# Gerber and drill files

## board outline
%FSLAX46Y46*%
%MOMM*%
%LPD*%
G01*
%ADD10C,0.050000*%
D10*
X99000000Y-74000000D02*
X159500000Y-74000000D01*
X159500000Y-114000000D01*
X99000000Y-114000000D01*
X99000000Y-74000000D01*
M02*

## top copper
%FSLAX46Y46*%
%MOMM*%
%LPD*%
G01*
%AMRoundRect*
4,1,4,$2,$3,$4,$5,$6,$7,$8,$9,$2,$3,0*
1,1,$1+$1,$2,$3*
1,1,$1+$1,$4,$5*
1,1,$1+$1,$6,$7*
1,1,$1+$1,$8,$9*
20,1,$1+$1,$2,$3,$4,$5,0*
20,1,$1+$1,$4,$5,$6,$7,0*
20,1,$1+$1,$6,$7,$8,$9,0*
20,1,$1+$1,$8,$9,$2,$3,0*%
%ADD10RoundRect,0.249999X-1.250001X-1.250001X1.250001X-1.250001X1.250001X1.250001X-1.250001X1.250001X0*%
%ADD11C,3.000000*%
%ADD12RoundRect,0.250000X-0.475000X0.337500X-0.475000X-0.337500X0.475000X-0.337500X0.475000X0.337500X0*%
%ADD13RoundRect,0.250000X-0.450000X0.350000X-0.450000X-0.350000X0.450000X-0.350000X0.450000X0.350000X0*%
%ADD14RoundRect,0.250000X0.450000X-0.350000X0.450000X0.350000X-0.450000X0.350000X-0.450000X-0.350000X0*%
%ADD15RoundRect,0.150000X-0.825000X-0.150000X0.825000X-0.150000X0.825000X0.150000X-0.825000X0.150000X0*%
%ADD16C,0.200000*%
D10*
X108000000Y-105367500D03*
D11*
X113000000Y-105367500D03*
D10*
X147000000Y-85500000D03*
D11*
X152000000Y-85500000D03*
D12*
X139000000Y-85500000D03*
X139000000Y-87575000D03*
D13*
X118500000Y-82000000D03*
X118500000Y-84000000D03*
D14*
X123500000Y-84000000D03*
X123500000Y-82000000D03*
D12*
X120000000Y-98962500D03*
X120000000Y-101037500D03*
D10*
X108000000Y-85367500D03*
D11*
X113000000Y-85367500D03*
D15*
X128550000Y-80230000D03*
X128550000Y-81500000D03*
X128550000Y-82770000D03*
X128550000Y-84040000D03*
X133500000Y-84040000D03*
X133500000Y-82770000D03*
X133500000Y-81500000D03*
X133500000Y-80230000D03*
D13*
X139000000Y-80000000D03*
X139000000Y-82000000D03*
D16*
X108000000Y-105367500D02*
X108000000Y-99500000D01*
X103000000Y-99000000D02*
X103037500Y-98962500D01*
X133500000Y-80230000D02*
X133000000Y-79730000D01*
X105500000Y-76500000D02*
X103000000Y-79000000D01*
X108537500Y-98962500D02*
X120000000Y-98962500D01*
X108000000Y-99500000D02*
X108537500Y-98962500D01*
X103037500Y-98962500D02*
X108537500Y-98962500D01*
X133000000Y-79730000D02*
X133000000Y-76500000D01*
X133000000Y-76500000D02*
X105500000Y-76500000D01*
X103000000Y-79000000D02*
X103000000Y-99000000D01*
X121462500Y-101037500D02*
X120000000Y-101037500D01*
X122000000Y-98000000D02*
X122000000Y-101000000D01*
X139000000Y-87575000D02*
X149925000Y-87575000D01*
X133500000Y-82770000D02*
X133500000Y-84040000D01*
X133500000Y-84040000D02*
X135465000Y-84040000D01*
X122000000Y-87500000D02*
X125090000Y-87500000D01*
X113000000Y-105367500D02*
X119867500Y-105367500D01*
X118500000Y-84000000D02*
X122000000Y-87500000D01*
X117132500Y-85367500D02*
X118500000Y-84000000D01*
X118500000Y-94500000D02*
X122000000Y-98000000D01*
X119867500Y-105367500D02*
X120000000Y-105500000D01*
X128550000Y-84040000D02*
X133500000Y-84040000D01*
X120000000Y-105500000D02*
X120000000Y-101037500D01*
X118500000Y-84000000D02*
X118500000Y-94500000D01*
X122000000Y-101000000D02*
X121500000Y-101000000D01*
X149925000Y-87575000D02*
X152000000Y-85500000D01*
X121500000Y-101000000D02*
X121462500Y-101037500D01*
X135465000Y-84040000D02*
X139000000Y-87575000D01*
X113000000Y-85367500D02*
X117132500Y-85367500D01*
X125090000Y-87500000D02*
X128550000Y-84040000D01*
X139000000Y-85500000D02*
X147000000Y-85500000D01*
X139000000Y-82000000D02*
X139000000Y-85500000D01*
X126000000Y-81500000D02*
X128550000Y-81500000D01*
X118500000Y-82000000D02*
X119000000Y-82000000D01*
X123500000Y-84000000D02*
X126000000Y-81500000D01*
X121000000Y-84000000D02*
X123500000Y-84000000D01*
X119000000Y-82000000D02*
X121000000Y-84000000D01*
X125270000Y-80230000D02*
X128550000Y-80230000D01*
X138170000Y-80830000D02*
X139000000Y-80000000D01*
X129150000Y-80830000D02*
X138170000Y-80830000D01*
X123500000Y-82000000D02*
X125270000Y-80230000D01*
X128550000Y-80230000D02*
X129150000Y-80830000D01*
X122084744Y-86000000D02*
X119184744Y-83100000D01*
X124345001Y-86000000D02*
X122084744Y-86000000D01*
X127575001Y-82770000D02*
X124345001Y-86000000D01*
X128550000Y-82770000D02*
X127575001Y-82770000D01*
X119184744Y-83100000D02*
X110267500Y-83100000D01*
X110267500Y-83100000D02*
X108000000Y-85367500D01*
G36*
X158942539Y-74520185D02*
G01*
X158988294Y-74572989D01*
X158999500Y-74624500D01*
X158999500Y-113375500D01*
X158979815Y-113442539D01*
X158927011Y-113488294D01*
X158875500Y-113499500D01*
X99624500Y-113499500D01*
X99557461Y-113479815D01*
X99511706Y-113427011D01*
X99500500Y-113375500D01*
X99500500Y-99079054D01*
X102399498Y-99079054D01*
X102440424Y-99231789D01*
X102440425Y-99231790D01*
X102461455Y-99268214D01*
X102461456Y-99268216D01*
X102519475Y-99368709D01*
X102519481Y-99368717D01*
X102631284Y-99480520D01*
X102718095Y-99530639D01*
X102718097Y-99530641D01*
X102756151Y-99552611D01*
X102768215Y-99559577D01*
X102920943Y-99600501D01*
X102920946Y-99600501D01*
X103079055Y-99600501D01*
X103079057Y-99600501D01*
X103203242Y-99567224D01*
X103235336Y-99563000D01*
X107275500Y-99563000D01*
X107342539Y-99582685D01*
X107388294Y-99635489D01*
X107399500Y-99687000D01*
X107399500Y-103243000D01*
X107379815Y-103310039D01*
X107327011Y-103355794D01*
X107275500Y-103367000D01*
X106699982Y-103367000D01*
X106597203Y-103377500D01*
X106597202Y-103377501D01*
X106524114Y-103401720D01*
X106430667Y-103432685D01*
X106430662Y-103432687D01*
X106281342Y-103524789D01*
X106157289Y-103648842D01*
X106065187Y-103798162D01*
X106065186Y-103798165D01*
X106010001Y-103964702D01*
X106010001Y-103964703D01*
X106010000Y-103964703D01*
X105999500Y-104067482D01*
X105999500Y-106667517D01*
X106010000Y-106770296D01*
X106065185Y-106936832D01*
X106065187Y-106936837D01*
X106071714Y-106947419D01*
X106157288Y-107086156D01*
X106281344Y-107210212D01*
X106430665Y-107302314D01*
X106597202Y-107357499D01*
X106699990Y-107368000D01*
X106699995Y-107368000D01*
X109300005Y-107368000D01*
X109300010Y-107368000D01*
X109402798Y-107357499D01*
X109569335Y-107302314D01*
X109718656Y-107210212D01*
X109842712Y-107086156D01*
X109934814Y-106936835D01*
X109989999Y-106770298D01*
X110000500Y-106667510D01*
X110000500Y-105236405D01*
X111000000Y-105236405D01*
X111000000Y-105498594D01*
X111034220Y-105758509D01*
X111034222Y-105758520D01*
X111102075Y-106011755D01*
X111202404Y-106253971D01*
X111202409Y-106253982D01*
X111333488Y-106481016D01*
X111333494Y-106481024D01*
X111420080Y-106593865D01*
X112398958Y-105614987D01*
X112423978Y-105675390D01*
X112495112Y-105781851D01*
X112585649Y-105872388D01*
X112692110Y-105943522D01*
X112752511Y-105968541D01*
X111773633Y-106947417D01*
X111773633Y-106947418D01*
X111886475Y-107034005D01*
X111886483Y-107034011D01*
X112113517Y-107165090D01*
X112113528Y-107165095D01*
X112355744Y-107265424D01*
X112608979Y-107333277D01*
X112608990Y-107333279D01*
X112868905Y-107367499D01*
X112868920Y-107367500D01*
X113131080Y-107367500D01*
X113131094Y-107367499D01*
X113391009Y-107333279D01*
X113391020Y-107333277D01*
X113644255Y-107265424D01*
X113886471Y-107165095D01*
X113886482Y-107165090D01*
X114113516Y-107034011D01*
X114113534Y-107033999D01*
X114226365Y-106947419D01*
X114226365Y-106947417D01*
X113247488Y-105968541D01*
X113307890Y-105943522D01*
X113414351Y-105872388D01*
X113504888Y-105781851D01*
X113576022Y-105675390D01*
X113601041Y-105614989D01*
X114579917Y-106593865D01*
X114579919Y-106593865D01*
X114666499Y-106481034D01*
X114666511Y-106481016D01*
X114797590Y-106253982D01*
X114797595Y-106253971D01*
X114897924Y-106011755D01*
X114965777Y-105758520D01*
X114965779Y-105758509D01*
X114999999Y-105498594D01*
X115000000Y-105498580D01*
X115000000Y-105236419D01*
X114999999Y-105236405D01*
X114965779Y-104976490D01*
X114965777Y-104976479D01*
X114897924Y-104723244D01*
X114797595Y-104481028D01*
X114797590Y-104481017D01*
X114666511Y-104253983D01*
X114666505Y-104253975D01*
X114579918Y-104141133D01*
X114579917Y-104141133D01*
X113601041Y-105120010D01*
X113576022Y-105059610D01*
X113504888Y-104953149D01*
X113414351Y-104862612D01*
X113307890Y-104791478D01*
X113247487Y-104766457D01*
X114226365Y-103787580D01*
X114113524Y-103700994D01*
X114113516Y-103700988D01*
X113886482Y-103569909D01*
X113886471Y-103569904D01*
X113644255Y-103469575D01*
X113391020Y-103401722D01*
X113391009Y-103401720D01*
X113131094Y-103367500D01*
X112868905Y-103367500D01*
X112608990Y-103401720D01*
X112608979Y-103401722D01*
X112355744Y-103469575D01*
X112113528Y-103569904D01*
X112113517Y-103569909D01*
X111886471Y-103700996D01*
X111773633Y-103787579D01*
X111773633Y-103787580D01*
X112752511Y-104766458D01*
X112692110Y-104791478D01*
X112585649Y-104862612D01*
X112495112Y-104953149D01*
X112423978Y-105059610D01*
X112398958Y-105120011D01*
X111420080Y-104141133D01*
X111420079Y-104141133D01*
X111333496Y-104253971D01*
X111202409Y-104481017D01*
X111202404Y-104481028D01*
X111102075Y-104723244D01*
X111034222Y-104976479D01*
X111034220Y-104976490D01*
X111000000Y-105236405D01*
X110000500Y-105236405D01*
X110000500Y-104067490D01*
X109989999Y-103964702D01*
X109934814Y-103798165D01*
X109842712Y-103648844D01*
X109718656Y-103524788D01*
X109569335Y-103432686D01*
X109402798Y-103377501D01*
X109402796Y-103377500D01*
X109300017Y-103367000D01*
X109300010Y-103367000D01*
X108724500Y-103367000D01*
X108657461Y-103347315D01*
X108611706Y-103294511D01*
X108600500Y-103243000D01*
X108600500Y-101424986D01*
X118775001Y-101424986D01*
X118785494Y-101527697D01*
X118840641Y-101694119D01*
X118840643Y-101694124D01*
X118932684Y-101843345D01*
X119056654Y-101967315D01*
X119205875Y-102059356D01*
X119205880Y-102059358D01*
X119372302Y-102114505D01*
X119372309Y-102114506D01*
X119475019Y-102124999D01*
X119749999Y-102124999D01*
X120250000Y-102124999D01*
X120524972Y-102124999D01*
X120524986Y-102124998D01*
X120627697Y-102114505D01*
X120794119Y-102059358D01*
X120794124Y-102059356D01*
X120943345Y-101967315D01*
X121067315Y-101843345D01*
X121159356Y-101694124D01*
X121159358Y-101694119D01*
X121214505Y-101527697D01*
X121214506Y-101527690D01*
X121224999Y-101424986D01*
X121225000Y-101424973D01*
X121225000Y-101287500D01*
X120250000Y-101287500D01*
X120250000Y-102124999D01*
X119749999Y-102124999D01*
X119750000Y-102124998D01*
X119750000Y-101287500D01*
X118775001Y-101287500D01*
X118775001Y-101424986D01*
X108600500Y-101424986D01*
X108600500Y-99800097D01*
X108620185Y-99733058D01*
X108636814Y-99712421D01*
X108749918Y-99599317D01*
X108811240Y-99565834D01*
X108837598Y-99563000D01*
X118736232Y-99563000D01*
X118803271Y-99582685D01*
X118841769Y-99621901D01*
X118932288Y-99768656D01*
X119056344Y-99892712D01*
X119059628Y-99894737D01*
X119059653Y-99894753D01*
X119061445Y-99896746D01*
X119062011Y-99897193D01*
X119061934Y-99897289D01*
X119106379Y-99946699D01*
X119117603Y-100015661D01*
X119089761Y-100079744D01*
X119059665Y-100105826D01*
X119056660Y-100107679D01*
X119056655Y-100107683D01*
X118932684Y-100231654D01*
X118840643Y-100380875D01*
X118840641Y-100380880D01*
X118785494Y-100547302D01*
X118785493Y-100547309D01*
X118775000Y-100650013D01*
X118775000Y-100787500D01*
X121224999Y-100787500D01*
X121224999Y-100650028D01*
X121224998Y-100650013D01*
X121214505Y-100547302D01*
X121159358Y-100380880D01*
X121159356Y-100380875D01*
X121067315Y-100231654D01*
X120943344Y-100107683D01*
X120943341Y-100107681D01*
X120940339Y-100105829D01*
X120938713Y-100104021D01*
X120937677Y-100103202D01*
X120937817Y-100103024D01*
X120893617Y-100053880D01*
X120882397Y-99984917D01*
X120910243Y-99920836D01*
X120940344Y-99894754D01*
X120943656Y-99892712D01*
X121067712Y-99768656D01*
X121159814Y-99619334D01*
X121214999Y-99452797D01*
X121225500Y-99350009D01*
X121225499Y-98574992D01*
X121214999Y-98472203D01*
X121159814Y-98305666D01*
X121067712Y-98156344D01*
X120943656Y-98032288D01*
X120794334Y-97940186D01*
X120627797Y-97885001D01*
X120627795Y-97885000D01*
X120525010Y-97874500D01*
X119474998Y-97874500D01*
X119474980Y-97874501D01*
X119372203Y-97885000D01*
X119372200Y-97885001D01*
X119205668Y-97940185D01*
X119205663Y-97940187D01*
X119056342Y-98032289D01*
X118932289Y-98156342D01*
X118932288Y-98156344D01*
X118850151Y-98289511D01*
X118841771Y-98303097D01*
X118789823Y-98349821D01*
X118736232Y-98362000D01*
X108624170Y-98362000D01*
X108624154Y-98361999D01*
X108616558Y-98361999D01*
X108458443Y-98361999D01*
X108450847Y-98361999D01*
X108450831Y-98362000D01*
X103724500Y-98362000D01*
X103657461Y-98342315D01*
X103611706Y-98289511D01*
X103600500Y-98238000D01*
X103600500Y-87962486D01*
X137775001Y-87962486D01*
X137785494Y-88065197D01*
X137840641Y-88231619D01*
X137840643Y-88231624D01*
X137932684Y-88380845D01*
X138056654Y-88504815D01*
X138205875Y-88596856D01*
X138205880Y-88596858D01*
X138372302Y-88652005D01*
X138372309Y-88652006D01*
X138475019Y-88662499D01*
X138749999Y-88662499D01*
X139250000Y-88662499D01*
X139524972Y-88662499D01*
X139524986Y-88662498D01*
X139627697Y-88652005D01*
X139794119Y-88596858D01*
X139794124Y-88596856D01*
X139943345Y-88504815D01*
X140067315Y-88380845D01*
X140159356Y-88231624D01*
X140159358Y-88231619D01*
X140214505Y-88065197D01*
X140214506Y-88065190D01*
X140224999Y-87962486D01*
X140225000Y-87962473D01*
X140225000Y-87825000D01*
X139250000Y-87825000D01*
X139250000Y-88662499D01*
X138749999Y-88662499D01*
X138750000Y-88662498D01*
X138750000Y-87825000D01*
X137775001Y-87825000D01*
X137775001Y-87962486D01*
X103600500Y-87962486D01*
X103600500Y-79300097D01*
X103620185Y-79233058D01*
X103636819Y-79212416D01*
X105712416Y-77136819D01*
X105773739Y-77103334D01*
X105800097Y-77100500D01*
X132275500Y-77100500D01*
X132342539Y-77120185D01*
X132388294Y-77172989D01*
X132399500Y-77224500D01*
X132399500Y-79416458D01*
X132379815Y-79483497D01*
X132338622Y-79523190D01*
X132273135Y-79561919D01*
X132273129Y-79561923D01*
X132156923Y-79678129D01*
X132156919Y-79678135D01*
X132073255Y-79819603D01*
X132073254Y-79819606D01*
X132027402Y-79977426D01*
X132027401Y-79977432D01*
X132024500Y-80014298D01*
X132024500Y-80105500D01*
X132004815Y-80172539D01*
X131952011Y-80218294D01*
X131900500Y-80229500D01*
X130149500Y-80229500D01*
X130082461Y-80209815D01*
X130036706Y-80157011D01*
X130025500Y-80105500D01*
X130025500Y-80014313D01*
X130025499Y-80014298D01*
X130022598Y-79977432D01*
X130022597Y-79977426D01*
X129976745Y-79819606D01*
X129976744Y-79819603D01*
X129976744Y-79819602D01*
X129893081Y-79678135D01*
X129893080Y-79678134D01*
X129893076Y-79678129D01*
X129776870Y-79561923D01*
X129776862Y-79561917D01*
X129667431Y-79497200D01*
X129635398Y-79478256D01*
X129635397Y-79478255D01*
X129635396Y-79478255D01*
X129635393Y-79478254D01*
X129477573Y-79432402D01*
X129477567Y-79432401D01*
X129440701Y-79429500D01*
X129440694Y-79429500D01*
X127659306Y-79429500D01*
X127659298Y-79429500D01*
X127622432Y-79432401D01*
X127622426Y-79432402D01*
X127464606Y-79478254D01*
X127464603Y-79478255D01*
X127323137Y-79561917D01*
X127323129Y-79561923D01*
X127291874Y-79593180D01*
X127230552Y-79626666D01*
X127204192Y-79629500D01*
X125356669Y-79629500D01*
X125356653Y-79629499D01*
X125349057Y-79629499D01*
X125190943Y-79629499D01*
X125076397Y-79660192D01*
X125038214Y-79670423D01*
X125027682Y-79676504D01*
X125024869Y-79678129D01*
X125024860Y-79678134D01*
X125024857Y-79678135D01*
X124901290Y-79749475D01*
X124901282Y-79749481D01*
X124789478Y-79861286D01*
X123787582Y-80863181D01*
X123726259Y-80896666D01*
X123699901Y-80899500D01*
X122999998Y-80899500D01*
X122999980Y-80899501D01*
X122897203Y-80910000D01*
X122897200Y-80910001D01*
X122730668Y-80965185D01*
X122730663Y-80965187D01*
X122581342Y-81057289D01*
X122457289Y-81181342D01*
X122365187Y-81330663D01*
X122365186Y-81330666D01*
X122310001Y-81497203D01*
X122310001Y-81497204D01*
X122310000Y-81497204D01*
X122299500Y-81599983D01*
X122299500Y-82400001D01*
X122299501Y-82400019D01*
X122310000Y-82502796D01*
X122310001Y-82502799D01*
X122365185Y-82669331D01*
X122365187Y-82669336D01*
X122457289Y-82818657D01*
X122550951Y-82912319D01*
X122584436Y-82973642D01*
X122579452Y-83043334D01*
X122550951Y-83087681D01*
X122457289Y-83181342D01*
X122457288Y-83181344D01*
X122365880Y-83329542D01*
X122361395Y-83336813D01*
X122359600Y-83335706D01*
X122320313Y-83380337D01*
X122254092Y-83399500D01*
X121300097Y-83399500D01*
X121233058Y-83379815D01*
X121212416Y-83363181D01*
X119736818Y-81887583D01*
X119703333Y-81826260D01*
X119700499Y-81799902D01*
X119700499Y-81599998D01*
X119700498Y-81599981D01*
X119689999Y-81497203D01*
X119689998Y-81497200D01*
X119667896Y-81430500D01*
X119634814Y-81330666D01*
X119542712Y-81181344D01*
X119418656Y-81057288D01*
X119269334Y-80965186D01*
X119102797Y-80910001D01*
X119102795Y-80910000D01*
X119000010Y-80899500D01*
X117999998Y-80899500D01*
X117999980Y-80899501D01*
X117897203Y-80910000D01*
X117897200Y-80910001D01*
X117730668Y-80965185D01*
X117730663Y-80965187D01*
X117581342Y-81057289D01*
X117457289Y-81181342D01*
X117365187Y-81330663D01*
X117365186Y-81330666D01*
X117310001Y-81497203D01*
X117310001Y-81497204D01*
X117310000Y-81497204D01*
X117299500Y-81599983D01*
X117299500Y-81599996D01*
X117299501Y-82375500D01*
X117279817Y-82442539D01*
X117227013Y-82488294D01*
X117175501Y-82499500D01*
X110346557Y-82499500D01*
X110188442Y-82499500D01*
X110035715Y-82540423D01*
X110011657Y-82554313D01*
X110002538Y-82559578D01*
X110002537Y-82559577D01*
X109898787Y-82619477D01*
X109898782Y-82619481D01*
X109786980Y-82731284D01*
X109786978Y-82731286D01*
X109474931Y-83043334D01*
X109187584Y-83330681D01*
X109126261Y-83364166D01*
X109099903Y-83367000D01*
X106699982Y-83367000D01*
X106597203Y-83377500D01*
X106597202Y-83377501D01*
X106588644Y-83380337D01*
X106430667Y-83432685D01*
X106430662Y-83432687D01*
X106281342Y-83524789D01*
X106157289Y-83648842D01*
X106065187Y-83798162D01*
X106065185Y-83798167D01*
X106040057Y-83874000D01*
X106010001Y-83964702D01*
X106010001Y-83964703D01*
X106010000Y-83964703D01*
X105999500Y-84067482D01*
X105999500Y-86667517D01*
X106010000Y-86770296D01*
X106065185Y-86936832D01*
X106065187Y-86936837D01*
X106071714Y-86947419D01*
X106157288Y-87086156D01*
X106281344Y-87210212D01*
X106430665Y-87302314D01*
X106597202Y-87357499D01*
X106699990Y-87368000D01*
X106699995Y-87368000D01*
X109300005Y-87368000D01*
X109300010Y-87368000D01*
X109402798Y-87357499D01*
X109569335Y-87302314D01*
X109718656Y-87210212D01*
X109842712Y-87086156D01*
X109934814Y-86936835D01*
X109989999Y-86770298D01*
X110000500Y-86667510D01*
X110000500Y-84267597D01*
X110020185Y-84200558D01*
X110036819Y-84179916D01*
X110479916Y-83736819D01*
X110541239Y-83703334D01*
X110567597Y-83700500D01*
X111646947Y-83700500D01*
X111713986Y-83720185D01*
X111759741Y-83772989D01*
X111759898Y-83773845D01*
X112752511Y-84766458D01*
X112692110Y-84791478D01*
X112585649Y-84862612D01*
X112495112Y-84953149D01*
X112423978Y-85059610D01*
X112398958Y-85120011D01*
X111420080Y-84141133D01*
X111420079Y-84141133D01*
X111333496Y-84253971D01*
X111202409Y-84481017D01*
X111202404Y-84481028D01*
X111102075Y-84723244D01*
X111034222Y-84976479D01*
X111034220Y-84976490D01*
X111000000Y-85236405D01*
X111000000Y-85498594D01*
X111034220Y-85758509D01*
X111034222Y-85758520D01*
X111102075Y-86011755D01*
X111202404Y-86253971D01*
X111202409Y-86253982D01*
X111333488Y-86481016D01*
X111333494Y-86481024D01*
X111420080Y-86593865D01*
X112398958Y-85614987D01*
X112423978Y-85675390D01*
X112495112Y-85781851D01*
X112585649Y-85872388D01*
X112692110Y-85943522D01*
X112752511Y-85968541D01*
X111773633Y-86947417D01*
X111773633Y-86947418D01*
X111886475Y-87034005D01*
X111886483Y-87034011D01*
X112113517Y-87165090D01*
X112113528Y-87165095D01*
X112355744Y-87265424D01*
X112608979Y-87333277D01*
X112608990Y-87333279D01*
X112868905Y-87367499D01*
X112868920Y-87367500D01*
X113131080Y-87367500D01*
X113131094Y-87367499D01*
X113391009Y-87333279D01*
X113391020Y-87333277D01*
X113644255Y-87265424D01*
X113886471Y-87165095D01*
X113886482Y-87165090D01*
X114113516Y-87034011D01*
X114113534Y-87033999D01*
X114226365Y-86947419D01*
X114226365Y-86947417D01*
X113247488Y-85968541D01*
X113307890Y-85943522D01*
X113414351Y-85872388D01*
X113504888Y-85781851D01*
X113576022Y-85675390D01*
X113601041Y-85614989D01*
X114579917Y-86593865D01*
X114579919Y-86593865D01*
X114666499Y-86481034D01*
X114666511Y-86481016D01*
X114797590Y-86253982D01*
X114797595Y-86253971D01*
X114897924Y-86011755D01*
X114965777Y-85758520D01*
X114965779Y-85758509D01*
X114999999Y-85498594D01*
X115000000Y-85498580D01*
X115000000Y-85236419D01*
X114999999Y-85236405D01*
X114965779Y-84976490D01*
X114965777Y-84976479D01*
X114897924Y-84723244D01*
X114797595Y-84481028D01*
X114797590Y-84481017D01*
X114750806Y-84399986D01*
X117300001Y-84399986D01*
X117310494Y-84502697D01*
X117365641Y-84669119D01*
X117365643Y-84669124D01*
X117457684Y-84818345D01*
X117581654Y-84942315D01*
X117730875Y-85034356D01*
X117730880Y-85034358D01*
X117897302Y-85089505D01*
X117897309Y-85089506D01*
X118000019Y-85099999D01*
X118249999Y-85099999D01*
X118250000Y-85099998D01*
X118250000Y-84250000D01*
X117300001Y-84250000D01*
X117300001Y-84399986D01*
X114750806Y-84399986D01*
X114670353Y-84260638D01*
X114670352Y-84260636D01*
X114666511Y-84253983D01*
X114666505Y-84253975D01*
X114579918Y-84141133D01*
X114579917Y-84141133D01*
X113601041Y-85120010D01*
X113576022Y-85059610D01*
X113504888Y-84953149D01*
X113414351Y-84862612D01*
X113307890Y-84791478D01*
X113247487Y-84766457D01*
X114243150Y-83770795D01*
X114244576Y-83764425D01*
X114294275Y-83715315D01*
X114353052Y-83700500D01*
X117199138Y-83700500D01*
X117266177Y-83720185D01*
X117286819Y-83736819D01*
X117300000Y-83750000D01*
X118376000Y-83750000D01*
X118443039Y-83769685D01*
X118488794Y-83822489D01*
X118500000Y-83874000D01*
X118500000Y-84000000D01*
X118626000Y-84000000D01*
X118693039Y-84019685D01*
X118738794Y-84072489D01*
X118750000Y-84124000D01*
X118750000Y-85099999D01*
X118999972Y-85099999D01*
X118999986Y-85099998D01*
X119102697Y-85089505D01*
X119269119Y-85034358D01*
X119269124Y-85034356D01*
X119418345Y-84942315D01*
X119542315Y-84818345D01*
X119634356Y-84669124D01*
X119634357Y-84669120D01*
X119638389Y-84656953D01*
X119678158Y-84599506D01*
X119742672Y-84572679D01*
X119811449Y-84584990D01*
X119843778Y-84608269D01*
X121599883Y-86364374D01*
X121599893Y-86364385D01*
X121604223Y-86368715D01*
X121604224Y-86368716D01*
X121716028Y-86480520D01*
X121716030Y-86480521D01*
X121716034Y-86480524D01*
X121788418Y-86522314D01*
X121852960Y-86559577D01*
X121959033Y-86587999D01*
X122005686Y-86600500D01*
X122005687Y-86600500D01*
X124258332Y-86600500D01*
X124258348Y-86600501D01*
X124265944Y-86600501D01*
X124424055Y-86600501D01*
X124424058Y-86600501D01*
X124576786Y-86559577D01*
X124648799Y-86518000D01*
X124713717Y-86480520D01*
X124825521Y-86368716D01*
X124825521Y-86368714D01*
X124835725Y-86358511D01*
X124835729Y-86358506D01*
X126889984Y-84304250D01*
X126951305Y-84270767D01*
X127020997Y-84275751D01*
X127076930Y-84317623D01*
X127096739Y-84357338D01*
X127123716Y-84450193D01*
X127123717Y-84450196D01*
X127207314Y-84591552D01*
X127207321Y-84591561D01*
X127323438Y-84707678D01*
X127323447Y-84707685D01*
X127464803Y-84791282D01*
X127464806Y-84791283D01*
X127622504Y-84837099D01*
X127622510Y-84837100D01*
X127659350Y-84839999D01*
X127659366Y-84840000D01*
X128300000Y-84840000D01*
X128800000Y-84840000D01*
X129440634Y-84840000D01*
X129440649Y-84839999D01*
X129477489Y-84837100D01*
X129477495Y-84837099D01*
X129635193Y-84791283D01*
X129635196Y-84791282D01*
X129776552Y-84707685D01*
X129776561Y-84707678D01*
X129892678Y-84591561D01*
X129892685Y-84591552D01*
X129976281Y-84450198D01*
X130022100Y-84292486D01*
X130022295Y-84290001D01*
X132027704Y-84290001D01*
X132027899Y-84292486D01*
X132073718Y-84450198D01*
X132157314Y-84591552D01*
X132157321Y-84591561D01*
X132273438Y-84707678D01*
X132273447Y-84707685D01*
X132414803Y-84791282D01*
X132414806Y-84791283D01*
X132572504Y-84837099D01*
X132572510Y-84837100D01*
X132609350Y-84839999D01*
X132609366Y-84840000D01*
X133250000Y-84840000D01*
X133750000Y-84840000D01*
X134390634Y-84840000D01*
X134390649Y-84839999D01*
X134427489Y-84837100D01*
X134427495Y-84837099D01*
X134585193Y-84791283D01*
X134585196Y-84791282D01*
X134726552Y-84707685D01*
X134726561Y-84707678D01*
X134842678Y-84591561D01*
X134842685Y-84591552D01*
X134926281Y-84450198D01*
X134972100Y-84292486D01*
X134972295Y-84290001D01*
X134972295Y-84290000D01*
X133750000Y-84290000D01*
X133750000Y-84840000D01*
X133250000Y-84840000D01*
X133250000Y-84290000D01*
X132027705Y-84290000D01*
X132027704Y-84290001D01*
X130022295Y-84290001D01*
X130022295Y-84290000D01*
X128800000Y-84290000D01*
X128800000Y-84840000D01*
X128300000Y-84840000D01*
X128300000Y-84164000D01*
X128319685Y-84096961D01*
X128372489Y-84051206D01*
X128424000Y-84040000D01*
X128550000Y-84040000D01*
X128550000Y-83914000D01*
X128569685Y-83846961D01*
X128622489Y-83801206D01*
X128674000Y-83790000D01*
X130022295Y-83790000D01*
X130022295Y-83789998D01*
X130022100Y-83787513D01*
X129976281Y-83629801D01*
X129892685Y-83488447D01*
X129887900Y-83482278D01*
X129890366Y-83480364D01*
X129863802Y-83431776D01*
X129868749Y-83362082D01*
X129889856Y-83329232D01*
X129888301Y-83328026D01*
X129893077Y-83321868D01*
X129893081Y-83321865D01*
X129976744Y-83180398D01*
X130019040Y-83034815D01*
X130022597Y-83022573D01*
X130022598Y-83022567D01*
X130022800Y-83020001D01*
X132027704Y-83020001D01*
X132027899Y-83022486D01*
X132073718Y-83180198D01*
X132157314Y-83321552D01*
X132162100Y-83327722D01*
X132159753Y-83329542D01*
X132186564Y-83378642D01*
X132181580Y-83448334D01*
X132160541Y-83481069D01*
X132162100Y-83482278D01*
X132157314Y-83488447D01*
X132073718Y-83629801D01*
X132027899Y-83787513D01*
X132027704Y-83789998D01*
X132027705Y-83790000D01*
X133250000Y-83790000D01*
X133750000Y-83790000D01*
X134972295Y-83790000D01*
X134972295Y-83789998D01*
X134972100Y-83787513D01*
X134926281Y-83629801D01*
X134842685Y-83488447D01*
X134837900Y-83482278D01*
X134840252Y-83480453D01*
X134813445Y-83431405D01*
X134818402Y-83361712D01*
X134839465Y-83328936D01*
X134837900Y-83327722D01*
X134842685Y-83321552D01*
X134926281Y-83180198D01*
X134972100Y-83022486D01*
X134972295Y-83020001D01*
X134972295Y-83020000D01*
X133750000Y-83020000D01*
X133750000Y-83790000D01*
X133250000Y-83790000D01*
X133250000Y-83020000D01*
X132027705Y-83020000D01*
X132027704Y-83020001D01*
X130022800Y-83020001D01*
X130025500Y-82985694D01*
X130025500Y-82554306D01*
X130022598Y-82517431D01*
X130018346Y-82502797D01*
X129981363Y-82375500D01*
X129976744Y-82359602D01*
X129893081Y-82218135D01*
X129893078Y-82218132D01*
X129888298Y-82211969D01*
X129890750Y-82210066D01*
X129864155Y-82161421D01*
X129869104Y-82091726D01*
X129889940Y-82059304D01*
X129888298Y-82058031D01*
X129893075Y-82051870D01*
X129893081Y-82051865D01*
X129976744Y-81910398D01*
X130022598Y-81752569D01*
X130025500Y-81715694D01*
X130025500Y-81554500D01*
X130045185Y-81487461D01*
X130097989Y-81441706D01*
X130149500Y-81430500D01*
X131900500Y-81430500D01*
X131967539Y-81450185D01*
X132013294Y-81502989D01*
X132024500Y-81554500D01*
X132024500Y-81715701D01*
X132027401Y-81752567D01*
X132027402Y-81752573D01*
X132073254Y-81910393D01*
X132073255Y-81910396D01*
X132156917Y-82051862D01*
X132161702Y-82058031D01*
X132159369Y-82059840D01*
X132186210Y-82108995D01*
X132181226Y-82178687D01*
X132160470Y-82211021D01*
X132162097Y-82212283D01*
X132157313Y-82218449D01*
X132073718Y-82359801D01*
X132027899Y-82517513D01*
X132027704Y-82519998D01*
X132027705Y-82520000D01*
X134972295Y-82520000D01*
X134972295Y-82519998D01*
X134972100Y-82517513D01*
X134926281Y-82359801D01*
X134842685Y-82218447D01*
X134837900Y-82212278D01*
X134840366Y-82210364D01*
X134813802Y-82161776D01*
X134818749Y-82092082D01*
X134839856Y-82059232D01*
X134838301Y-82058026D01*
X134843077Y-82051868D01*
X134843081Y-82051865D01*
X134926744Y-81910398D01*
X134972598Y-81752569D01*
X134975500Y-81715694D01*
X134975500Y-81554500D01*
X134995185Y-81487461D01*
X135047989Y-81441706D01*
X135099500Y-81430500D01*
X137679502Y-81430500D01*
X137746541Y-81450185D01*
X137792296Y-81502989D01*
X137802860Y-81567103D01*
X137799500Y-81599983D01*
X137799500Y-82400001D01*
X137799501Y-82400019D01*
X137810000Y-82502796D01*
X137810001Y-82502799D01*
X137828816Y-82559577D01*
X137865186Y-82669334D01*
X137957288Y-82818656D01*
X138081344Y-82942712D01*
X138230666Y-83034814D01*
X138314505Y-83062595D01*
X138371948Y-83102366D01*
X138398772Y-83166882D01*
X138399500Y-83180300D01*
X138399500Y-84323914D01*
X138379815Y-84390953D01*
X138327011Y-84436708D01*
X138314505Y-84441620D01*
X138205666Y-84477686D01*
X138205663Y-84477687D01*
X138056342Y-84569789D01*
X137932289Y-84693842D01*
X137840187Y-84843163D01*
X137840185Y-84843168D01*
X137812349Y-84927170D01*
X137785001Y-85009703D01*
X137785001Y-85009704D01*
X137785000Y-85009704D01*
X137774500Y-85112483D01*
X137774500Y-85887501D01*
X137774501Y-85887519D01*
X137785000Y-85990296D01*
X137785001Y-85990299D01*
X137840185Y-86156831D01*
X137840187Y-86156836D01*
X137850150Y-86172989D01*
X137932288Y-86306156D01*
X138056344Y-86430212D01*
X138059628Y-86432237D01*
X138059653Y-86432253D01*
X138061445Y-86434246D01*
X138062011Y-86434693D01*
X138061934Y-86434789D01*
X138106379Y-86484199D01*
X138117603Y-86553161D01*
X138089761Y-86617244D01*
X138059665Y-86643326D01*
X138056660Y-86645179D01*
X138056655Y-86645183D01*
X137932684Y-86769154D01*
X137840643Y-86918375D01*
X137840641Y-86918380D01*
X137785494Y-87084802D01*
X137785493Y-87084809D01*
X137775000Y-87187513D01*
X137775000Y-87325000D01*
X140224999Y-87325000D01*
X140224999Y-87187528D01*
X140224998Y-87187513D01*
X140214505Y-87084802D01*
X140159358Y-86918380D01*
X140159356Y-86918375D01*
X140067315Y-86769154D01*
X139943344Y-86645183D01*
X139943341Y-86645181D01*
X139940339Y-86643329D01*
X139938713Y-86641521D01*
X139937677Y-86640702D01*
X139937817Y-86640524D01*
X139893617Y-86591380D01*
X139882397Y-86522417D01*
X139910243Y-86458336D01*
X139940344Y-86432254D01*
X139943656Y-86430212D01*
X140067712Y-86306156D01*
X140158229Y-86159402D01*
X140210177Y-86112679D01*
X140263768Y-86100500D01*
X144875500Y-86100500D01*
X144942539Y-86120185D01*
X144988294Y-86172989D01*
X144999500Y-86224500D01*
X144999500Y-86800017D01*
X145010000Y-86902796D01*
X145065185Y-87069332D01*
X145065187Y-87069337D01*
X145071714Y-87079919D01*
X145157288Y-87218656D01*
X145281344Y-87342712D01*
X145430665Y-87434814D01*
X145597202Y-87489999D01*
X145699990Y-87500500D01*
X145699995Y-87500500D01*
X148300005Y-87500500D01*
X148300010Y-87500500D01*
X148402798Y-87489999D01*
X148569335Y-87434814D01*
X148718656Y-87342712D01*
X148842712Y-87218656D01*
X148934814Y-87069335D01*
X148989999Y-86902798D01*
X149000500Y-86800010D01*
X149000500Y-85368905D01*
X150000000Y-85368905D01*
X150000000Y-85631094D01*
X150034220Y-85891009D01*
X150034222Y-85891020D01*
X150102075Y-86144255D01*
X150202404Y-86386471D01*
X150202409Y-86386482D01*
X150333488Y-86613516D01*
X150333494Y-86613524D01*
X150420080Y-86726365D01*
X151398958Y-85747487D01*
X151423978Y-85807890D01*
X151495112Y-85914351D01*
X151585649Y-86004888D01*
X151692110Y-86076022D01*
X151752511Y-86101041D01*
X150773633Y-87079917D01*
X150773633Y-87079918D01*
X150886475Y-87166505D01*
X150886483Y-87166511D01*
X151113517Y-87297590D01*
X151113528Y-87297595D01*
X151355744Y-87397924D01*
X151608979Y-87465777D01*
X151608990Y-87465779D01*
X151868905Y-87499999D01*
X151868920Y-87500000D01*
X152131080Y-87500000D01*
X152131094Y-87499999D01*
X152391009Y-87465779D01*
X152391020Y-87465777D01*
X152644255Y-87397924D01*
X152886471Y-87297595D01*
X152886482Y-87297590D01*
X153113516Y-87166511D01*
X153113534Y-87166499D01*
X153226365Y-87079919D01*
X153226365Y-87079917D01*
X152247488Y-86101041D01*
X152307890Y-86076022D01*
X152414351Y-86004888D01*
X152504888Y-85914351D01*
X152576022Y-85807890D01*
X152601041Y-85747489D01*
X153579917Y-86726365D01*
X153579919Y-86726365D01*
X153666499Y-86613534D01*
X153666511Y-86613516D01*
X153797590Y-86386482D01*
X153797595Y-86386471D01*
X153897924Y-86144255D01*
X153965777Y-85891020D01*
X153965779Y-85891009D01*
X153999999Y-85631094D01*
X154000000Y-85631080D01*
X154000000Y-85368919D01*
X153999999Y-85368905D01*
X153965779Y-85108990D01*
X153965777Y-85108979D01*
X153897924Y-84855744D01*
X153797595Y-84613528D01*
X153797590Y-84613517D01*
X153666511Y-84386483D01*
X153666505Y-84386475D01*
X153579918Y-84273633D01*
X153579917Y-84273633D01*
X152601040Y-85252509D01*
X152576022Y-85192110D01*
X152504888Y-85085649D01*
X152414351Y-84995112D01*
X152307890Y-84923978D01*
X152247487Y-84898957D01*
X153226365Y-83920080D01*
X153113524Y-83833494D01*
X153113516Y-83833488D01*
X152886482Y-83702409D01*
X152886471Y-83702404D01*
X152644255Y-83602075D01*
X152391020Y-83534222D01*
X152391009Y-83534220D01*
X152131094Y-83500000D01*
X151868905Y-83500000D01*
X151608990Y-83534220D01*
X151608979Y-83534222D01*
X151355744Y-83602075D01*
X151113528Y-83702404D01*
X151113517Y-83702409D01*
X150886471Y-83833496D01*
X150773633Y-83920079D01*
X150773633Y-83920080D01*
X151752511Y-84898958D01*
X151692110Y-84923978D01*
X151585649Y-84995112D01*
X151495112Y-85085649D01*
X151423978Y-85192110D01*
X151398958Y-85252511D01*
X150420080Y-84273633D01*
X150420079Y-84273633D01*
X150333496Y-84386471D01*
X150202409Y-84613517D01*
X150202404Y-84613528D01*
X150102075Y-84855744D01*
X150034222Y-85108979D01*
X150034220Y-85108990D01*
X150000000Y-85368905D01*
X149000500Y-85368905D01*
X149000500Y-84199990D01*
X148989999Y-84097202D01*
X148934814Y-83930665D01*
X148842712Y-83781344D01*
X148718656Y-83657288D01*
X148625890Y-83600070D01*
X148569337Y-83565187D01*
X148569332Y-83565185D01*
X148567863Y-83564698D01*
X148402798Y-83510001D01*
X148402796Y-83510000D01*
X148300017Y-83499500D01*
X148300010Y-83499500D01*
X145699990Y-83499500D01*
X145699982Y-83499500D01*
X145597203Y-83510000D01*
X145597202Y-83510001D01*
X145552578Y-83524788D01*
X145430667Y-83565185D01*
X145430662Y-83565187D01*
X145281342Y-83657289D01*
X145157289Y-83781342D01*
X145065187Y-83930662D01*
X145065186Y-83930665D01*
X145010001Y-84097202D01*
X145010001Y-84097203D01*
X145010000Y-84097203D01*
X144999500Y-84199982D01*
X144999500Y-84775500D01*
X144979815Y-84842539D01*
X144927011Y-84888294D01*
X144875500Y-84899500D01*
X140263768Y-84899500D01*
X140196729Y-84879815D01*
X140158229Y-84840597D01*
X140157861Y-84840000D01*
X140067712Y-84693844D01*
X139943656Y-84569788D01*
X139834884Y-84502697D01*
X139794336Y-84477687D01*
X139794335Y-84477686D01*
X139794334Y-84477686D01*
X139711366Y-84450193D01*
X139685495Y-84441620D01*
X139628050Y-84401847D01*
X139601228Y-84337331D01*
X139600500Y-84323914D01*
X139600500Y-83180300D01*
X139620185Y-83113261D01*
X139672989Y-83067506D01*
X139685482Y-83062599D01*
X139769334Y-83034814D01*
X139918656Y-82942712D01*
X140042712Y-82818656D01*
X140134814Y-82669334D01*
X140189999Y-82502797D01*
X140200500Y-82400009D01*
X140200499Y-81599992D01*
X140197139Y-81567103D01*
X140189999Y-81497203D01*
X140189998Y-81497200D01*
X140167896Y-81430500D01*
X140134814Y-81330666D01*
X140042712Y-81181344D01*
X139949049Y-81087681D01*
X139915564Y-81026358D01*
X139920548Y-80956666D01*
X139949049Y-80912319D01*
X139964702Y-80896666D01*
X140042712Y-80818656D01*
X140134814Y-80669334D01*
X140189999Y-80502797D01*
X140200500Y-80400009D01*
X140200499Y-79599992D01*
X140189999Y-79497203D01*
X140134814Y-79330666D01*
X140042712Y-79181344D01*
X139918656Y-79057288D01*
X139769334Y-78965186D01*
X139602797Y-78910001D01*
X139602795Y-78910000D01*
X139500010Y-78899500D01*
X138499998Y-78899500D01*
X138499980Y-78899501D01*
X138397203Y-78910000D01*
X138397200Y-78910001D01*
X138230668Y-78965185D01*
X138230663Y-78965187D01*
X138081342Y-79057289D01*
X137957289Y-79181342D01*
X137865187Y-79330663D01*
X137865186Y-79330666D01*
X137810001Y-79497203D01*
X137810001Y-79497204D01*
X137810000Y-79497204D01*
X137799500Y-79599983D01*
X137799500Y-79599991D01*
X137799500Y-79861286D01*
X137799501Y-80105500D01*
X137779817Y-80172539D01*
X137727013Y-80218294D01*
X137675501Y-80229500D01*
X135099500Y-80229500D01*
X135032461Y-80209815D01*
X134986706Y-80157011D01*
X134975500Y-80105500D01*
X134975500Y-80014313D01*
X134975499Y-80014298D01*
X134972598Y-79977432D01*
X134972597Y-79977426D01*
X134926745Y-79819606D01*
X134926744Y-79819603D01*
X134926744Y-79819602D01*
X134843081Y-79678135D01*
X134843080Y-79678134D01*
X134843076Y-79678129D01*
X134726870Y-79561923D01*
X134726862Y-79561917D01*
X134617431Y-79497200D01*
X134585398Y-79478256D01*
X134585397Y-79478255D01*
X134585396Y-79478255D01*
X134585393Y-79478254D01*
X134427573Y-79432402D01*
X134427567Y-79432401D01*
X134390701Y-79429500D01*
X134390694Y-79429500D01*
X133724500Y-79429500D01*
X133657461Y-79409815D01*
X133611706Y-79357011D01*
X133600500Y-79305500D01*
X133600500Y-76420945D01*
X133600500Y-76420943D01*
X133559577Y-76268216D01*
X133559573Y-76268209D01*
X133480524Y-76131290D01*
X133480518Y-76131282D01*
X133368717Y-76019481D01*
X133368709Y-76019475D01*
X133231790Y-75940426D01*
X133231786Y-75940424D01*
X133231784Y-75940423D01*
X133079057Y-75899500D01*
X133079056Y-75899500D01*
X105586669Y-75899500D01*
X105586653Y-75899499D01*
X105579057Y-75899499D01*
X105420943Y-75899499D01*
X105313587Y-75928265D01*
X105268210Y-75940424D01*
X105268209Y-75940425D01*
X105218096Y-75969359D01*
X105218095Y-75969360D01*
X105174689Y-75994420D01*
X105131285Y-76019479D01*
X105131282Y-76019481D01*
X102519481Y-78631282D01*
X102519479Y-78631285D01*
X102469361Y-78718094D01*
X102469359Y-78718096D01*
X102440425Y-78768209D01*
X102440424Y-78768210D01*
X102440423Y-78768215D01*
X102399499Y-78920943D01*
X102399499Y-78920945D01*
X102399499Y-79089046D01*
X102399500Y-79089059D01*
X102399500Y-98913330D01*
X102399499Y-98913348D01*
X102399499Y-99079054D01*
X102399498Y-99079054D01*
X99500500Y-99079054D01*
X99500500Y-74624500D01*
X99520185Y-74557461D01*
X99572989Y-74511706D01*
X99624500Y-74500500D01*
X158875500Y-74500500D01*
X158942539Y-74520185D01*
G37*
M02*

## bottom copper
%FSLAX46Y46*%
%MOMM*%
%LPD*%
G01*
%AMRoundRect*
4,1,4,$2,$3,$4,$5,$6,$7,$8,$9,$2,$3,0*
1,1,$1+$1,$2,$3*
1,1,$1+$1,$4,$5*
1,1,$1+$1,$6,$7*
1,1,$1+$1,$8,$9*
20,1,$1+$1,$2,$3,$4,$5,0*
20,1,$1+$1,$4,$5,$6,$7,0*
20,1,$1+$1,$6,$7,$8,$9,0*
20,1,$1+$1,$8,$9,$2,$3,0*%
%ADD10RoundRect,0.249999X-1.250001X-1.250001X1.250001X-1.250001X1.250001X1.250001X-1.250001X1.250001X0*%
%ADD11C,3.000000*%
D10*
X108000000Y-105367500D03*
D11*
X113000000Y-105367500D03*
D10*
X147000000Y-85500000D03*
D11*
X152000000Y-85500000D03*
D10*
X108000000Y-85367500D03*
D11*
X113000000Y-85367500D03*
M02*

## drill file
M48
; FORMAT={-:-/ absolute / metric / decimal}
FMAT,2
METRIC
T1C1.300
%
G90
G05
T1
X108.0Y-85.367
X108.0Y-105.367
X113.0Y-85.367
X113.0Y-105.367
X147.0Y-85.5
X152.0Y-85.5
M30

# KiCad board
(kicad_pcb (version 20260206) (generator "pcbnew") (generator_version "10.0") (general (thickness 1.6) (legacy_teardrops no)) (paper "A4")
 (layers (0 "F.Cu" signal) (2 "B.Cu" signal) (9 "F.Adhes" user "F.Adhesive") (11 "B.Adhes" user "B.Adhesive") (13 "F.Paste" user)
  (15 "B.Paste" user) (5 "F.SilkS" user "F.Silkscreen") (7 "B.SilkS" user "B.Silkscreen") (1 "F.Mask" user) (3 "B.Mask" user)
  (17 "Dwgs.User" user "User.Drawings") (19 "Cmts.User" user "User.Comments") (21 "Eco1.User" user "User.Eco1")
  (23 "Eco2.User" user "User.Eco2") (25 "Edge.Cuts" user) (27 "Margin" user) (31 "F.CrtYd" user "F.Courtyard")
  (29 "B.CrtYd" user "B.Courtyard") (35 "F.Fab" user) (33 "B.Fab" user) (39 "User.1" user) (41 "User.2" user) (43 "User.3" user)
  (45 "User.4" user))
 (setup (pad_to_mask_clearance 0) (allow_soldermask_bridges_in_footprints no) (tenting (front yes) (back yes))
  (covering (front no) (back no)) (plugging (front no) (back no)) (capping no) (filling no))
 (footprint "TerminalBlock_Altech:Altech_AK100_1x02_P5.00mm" (layer "F.Cu") (at 108 105.3675)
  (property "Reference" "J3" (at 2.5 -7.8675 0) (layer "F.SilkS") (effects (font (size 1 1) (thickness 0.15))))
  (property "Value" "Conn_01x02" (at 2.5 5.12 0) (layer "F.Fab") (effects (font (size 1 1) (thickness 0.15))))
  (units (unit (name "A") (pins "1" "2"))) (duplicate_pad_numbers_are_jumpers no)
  (pad "1" thru_hole roundrect (at 0 0) (size 3 3) (drill 1.3) (layers "*.Cu" "*.Mask") (remove_unused_layers no)
   (roundrect_rratio 0.083333) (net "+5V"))
  (pad "2" thru_hole circle (at 5 0) (size 3 3) (drill 1.3) (layers "*.Cu" "*.Mask") (remove_unused_layers no) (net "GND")))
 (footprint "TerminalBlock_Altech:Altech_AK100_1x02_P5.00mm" (layer "F.Cu") (at 147 85.5)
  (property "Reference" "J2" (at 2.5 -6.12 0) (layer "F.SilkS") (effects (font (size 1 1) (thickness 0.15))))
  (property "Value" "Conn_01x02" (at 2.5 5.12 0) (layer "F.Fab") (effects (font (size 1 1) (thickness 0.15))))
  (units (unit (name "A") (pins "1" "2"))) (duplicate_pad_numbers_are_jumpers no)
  (pad "1" thru_hole roundrect (at 0 0) (size 3 3) (drill 1.3) (layers "*.Cu" "*.Mask") (remove_unused_layers no)
   (roundrect_rratio 0.083333) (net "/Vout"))
  (pad "2" thru_hole circle (at 5 0) (size 3 3) (drill 1.3) (layers "*.Cu" "*.Mask") (remove_unused_layers no) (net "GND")))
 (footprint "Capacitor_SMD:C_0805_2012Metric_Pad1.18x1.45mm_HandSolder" (layer "F.Cu") (at 139 86.5375 -90)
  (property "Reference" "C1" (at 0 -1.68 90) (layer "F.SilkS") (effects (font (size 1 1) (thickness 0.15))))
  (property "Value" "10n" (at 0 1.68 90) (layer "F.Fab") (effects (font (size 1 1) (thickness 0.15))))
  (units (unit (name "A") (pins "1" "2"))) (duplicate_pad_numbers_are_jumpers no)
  (pad "1" smd roundrect (at -1.0375 0 270) (size 1.175 1.45) (layers "F.Cu" "F.Mask" "F.Paste") (roundrect_rratio 0.212766) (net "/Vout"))
  (pad "2" smd roundrect (at 1.0375 0 270) (size 1.175 1.45) (layers "F.Cu" "F.Mask" "F.Paste") (roundrect_rratio 0.212766) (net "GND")))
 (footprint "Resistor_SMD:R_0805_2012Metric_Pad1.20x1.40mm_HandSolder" (layer "F.Cu") (at 118.5 83 -90)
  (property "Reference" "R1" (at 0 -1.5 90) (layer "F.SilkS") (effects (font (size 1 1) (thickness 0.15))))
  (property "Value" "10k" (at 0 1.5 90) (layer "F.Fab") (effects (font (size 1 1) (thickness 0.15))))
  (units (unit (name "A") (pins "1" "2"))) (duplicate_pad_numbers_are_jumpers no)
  (pad "1" smd roundrect (at -1 0 270) (size 1.2 1.4) (layers "F.Cu" "F.Mask" "F.Paste") (roundrect_rratio 0.208333) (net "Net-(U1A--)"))
  (pad "2" smd roundrect (at 1 0 270) (size 1.2 1.4) (layers "F.Cu" "F.Mask" "F.Paste") (roundrect_rratio 0.208333) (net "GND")))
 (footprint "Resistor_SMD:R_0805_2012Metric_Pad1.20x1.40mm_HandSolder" (layer "F.Cu") (at 123.5 83 90)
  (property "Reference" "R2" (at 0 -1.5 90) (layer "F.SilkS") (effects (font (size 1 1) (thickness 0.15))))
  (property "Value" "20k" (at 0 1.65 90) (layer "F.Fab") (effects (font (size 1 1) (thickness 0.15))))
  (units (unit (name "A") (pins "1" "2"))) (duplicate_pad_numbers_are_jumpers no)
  (pad "1" smd roundrect (at -1 0 90) (size 1.2 1.4) (layers "F.Cu" "F.Mask" "F.Paste") (roundrect_rratio 0.208333) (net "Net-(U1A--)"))
  (pad "2" smd roundrect (at 1 0 90) (size 1.2 1.4) (layers "F.Cu" "F.Mask" "F.Paste") (roundrect_rratio 0.208333) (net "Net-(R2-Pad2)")))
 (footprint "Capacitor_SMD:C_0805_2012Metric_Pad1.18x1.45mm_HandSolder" (layer "F.Cu") (at 120 100 -90)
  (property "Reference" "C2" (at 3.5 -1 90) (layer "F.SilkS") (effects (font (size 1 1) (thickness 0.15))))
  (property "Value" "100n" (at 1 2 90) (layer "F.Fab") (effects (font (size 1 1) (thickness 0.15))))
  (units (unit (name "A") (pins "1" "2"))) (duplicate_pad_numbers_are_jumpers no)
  (pad "1" smd roundrect (at -1.0375 0 270) (size 1.175 1.45) (layers "F.Cu" "F.Mask" "F.Paste") (roundrect_rratio 0.212766) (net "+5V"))
  (pad "2" smd roundrect (at 1.0375 0 270) (size 1.175 1.45) (layers "F.Cu" "F.Mask" "F.Paste") (roundrect_rratio 0.212766) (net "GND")))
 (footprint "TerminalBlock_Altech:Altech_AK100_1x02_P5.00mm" (layer "F.Cu") (at 108 85.3675)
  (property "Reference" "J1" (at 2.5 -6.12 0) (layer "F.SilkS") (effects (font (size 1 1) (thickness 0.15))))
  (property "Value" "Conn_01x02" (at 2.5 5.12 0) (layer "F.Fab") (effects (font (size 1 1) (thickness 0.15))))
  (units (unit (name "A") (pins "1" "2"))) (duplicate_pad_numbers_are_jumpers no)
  (pad "1" thru_hole roundrect (at 0 0) (size 3 3) (drill 1.3) (layers "*.Cu" "*.Mask") (remove_unused_layers no)
   (roundrect_rratio 0.083333) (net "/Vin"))
  (pad "2" thru_hole circle (at 5 0) (size 3 3) (drill 1.3) (layers "*.Cu" "*.Mask") (remove_unused_layers no) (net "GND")))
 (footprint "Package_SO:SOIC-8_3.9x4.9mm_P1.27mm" (layer "F.Cu") (at 131.025 82.135)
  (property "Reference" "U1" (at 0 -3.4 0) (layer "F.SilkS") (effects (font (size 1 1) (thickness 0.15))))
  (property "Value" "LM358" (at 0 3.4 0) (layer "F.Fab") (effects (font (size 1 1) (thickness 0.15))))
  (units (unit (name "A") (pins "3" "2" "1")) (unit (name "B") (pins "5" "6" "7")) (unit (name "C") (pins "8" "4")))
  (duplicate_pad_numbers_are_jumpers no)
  (pad "1" smd roundrect (at -2.475 -1.905) (size 1.95 0.6) (layers "F.Cu" "F.Mask" "F.Paste") (roundrect_rratio 0.25) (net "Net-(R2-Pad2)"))
  (pad "2" smd roundrect (at -2.475 -0.635) (size 1.95 0.6) (layers "F.Cu" "F.Mask" "F.Paste") (roundrect_rratio 0.25) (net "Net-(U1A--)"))
  (pad "3" smd roundrect (at -2.475 0.635) (size 1.95 0.6) (layers "F.Cu" "F.Mask" "F.Paste") (roundrect_rratio 0.25) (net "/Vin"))
  (pad "4" smd roundrect (at -2.475 1.905) (size 1.95 0.6) (layers "F.Cu" "F.Mask" "F.Paste") (roundrect_rratio 0.25) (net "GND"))
  (pad "5" smd roundrect (at 2.475 1.905) (size 1.95 0.6) (layers "F.Cu" "F.Mask" "F.Paste") (roundrect_rratio 0.25) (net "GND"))
  (pad "6" smd roundrect (at 2.475 0.635) (size 1.95 0.6) (layers "F.Cu" "F.Mask" "F.Paste") (roundrect_rratio 0.25) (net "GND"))
  (pad "7" smd roundrect (at 2.475 -0.635) (size 1.95 0.6) (layers "F.Cu" "F.Mask" "F.Paste") (roundrect_rratio 0.25)
   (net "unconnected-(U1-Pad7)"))
  (pad "8" smd roundrect (at 2.475 -1.905) (size 1.95 0.6) (layers "F.Cu" "F.Mask" "F.Paste") (roundrect_rratio 0.25) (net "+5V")))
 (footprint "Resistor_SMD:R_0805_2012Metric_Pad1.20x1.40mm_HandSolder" (layer "F.Cu") (at 139 81 -90)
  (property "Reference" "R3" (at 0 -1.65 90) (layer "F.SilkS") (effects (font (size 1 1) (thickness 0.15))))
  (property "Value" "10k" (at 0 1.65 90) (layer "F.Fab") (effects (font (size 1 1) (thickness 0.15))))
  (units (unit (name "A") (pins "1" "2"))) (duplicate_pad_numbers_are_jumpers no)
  (pad "1" smd roundrect (at -1 0 270) (size 1.2 1.4) (layers "F.Cu" "F.Mask" "F.Paste") (roundrect_rratio 0.208333) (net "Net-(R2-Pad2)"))
  (pad "2" smd roundrect (at 1 0 270) (size 1.2 1.4) (layers "F.Cu" "F.Mask" "F.Paste") (roundrect_rratio 0.208333) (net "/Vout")))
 (gr_rect (start 99 74) (end 159.5 114) (stroke (width 0.05) (type default)) (fill no) (layer "Edge.Cuts"))
 (segment (start 108 105.3675) (end 108 99.5) (width 0.2) (layer "F.Cu") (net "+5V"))
 (segment (start 103 99) (end 103.0375 98.9625) (width 0.2) (layer "F.Cu") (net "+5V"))
 (segment (start 133.5 80.23) (end 133 79.73) (width 0.2) (layer "F.Cu") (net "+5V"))
 (segment (start 105.5 76.5) (end 103 79) (width 0.2) (layer "F.Cu") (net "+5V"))
 (segment (start 108.5375 98.9625) (end 120 98.9625) (width 0.2) (layer "F.Cu") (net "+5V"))
 (segment (start 108 99.5) (end 108.5375 98.9625) (width 0.2) (layer "F.Cu") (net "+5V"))
 (segment (start 103.0375 98.9625) (end 108.5375 98.9625) (width 0.2) (layer "F.Cu") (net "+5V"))
 (segment (start 133 79.73) (end 133 76.5) (width 0.2) (layer "F.Cu") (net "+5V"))
 (segment (start 133 76.5) (end 105.5 76.5) (width 0.2) (layer "F.Cu") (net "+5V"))
 (segment (start 103 79) (end 103 99) (width 0.2) (layer "F.Cu") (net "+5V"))
 (segment (start 121.4625 101.0375) (end 120 101.0375) (width 0.2) (layer "F.Cu") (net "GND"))
 (segment (start 122 98) (end 122 101) (width 0.2) (layer "F.Cu") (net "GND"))
 (segment (start 139 87.575) (end 149.925 87.575) (width 0.2) (layer "F.Cu") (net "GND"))
 (segment (start 133.5 82.77) (end 133.5 84.04) (width 0.2) (layer "F.Cu") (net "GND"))
 (segment (start 133.5 84.04) (end 135.465 84.04) (width 0.2) (layer "F.Cu") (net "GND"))
 (segment (start 122 87.5) (end 125.09 87.5) (width 0.2) (layer "F.Cu") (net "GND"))
 (segment (start 113 105.3675) (end 119.8675 105.3675) (width 0.2) (layer "F.Cu") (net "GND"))
 (segment (start 118.5 84) (end 122 87.5) (width 0.2) (layer "F.Cu") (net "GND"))
 (segment (start 117.1325 85.3675) (end 118.5 84) (width 0.2) (layer "F.Cu") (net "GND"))
 (segment (start 118.5 94.5) (end 122 98) (width 0.2) (layer "F.Cu") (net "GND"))
 (segment (start 119.8675 105.3675) (end 120 105.5) (width 0.2) (layer "F.Cu") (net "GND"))
 (segment (start 128.55 84.04) (end 133.5 84.04) (width 0.2) (layer "F.Cu") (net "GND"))
 (segment (start 120 105.5) (end 120 101.0375) (width 0.2) (layer "F.Cu") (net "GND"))
 (segment (start 118.5 84) (end 118.5 94.5) (width 0.2) (layer "F.Cu") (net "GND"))
 (segment (start 122 101) (end 121.5 101) (width 0.2) (layer "F.Cu") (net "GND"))
 (segment (start 149.925 87.575) (end 152 85.5) (width 0.2) (layer "F.Cu") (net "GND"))
 (segment (start 121.5 101) (end 121.4625 101.0375) (width 0.2) (layer "F.Cu") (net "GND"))
 (segment (start 135.465 84.04) (end 139 87.575) (width 0.2) (layer "F.Cu") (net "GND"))
 (segment (start 113 85.3675) (end 117.1325 85.3675) (width 0.2) (layer "F.Cu") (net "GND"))
 (segment (start 125.09 87.5) (end 128.55 84.04) (width 0.2) (layer "F.Cu") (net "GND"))
 (segment (start 139 85.5) (end 147 85.5) (width 0.2) (layer "F.Cu") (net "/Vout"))
 (segment (start 139 82) (end 139 85.5) (width 0.2) (layer "F.Cu") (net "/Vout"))
 (segment (start 126 81.5) (end 128.55 81.5) (width 0.2) (layer "F.Cu") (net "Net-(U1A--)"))
 (segment (start 118.5 82) (end 119 82) (width 0.2) (layer "F.Cu") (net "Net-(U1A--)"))
 (segment (start 123.5 84) (end 126 81.5) (width 0.2) (layer "F.Cu") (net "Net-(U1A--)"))
 (segment (start 121 84) (end 123.5 84) (width 0.2) (layer "F.Cu") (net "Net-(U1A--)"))
 (segment (start 119 82) (end 121 84) (width 0.2) (layer "F.Cu") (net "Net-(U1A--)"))
 (segment (start 125.27 80.23) (end 128.55 80.23) (width 0.2) (layer "F.Cu") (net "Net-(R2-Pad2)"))
 (segment (start 138.17 80.83) (end 139 80) (width 0.2) (layer "F.Cu") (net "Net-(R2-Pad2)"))
 (segment (start 129.15 80.83) (end 138.17 80.83) (width 0.2) (layer "F.Cu") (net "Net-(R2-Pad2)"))
 (segment (start 123.5 82) (end 125.27 80.23) (width 0.2) (layer "F.Cu") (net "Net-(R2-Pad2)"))
 (segment (start 128.55 80.23) (end 129.15 80.83) (width 0.2) (layer "F.Cu") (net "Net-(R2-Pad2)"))
 (segment (start 122.084744 86) (end 119.184744 83.1) (width 0.2) (layer "F.Cu") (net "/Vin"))
 (segment (start 124.345001 86) (end 122.084744 86) (width 0.2) (layer "F.Cu") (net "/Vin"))
 (segment (start 127.575001 82.77) (end 124.345001 86) (width 0.2) (layer "F.Cu") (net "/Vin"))
 (segment (start 128.55 82.77) (end 127.575001 82.77) (width 0.2) (layer "F.Cu") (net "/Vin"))
 (segment (start 119.184744 83.1) (end 110.2675 83.1) (width 0.2) (layer "F.Cu") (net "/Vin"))
 (segment (start 110.2675 83.1) (end 108 85.3675) (width 0.2) (layer "F.Cu") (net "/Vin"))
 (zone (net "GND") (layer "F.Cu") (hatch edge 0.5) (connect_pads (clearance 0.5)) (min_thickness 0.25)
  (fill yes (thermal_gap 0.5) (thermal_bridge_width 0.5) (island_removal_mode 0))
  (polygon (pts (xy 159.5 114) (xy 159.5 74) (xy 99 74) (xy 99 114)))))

